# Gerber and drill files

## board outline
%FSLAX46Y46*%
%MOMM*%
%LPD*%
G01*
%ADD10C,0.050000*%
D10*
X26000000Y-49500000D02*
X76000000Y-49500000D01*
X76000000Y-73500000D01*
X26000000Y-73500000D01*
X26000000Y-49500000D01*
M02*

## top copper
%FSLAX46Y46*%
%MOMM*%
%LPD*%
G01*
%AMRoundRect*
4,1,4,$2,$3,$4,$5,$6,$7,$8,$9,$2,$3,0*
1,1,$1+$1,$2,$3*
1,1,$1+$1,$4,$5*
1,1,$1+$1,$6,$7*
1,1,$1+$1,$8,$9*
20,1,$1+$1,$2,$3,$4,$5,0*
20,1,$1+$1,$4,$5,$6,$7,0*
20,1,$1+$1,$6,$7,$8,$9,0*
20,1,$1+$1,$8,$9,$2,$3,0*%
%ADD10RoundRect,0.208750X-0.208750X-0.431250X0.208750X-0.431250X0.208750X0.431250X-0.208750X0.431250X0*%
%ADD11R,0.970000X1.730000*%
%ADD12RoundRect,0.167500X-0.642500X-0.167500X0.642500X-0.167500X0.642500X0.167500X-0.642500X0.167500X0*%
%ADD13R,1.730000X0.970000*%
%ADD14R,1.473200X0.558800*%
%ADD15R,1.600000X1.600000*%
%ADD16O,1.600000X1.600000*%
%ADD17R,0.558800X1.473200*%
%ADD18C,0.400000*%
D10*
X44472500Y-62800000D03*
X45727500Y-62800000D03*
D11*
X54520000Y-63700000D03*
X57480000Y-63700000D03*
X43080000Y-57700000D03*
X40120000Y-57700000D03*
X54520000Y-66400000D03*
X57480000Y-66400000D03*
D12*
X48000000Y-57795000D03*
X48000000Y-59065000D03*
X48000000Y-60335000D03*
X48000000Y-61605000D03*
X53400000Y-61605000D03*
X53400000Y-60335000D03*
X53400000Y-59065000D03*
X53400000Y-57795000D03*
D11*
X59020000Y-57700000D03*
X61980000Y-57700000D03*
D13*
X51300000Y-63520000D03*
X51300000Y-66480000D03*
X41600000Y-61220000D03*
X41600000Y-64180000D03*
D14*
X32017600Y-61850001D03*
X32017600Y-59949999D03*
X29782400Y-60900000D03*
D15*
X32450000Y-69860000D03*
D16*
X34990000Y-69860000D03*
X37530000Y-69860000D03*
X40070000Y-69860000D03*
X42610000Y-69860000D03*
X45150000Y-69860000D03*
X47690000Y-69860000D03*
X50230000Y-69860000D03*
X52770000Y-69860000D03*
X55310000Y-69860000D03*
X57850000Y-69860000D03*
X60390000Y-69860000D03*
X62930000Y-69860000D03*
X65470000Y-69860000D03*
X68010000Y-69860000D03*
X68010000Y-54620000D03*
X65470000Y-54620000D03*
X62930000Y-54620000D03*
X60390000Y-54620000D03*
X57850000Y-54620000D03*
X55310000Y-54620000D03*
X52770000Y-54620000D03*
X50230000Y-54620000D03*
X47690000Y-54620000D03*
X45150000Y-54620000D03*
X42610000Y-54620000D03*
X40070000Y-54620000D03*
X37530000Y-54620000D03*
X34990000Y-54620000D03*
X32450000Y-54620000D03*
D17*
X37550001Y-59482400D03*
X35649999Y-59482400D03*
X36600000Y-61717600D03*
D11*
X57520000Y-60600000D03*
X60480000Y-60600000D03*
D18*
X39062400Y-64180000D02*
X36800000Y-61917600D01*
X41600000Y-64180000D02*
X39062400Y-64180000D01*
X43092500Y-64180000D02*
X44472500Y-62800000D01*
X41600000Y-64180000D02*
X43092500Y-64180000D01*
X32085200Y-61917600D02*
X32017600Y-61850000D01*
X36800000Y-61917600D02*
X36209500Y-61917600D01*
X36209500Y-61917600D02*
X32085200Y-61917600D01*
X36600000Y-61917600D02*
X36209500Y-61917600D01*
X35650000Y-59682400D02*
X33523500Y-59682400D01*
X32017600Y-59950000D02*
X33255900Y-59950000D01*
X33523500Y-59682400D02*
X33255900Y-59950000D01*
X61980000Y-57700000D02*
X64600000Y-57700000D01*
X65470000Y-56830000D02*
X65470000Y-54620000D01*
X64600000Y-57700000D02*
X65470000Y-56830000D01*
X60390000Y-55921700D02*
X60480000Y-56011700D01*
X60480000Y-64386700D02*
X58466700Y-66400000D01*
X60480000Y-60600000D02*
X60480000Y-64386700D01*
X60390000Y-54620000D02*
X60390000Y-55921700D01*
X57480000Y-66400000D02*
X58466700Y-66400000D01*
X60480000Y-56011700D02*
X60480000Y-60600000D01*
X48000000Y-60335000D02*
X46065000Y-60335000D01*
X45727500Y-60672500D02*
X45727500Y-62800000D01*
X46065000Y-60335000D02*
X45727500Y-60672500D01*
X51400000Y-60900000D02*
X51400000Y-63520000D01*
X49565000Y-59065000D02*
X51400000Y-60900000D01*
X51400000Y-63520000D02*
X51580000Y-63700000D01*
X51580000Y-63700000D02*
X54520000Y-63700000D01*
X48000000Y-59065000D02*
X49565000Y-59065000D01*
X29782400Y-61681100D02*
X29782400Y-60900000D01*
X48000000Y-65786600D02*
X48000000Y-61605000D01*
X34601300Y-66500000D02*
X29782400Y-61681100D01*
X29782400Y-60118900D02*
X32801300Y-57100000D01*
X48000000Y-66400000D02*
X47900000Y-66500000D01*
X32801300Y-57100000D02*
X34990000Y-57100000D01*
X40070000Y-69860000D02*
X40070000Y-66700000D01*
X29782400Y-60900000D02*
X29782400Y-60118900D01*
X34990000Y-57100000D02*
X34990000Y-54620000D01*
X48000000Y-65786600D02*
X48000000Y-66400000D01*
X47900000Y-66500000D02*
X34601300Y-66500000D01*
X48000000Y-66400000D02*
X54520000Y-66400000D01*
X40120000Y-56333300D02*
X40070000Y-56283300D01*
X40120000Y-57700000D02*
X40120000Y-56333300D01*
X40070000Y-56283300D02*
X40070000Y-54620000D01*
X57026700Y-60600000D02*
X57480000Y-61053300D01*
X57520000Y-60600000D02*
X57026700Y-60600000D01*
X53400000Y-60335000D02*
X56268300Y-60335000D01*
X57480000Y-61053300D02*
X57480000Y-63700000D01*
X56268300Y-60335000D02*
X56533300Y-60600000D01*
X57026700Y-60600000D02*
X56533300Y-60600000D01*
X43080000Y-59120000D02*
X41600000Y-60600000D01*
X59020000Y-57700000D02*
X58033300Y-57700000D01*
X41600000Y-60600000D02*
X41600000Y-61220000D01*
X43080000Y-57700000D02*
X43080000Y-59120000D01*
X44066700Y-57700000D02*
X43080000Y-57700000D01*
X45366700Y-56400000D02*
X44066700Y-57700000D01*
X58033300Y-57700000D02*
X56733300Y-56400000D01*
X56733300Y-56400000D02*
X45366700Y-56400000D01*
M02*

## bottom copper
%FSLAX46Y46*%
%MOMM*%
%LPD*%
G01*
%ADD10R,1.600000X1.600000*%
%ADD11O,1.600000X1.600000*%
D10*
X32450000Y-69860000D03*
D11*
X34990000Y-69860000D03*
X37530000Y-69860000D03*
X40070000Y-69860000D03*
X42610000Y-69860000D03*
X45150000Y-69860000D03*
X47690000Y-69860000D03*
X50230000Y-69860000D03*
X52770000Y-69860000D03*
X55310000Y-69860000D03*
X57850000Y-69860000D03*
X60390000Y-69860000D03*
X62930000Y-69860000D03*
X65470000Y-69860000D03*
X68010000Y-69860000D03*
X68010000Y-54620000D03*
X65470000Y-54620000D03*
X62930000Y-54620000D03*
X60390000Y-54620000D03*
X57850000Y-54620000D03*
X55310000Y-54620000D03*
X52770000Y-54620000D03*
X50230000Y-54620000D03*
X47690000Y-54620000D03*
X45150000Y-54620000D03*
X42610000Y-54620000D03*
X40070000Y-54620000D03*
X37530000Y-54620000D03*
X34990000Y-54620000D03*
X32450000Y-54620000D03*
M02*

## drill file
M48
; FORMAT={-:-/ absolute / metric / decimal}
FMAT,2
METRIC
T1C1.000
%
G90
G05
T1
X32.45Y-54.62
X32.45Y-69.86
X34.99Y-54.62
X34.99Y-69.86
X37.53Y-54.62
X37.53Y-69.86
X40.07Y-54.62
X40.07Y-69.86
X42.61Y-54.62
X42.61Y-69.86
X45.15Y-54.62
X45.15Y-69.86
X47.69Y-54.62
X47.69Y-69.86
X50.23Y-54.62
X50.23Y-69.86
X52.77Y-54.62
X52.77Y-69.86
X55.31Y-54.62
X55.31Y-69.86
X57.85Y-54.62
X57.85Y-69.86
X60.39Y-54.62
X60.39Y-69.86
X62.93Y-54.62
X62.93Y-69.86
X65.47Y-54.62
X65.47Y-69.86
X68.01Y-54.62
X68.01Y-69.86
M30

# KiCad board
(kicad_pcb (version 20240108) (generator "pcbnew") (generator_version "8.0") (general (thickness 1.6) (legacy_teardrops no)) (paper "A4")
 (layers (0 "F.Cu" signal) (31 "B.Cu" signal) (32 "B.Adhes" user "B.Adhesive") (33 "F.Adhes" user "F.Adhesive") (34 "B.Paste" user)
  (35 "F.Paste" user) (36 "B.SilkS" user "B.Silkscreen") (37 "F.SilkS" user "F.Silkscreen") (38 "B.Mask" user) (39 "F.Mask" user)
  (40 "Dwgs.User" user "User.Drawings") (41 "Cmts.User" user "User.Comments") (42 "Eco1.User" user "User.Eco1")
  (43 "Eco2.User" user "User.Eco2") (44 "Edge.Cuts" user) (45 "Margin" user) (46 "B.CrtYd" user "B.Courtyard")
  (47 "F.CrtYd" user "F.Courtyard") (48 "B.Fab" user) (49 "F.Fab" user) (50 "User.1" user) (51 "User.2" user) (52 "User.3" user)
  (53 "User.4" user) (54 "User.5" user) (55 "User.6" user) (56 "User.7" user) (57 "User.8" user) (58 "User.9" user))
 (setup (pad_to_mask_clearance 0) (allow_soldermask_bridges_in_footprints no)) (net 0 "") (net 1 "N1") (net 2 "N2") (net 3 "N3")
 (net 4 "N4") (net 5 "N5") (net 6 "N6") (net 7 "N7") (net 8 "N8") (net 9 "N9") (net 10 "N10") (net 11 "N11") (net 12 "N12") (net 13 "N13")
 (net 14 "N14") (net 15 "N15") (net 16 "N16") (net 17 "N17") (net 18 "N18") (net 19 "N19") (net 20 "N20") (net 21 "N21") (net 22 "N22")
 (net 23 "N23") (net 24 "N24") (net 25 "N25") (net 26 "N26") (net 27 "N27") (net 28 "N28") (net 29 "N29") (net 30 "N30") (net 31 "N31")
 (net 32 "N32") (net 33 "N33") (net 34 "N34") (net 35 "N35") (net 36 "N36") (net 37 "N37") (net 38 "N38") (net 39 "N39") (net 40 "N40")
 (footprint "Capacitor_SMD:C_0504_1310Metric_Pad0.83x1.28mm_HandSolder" (layer "F.Cu") (at 45.1 62.8)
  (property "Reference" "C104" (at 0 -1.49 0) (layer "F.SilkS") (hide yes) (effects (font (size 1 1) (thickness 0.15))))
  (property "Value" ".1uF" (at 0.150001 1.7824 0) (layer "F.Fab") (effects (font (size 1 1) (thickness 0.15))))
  (pad "1" smd roundrect (at -0.6275 0) (size 0.835 1.28) (layers "F.Cu" "F.Paste" "F.Mask") (roundrect_rratio 0.25) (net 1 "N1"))
  (pad "2" smd roundrect (at 0.6275 0) (size 0.835 1.28) (layers "F.Cu" "F.Paste" "F.Mask") (roundrect_rratio 0.25) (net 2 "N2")))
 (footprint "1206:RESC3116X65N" (layer "F.Cu") (at 56 63.7)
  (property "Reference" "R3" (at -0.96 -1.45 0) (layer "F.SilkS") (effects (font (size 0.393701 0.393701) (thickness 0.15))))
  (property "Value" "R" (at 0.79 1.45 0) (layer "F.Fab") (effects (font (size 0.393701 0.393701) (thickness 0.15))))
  (pad "1" smd rect (at -1.48 0) (size 0.97 1.73) (layers "F.Cu" "F.Paste" "F.Mask") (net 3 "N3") (solder_mask_margin 0.102))
  (pad "2" smd rect (at 1.48 0) (size 0.97 1.73) (layers "F.Cu" "F.Paste" "F.Mask") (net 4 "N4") (solder_mask_margin 0.102)))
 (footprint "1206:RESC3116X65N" (layer "F.Cu") (at 41.6 57.7 180)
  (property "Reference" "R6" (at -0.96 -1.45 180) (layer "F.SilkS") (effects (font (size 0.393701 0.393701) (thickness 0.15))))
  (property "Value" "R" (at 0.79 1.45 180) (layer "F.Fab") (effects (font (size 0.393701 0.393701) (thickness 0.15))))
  (pad "1" smd rect (at -1.48 0 180) (size 0.97 1.73) (layers "F.Cu" "F.Paste" "F.Mask") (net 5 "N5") (solder_mask_margin 0.102))
  (pad "2" smd rect (at 1.48 0 180) (size 0.97 1.73) (layers "F.Cu" "F.Paste" "F.Mask") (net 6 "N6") (solder_mask_margin 0.102)))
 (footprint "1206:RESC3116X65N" (layer "F.Cu") (at 56 66.4)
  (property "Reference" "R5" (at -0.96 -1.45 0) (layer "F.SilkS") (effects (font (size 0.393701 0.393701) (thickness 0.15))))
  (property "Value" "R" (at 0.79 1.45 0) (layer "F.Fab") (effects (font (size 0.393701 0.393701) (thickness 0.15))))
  (pad "1" smd rect (at -1.48 0) (size 0.97 1.73) (layers "F.Cu" "F.Paste" "F.Mask") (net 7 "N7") (solder_mask_margin 0.102))
  (pad "2" smd rect (at 1.48 0) (size 0.97 1.73) (layers "F.Cu" "F.Paste" "F.Mask") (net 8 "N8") (solder_mask_margin 0.102)))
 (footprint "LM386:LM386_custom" (layer "F.Cu") (at 48 57.795)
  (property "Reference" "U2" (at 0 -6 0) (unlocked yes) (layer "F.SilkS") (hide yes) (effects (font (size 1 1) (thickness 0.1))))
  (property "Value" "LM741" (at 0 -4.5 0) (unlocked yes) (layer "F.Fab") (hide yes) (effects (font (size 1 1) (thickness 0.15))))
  (pad "1" smd roundrect (at 0 0) (size 1.62 0.67) (layers "F.Cu" "F.Paste" "F.Mask") (roundrect_rratio 0.25) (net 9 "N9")
   (thermal_bridge_angle 45))
  (pad "2" smd roundrect (at 0 1.27) (size 1.62 0.67) (layers "F.Cu" "F.Paste" "F.Mask") (roundrect_rratio 0.25) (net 3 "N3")
   (thermal_bridge_angle 45))
  (pad "3" smd roundrect (at 0 2.54) (size 1.62 0.67) (layers "F.Cu" "F.Paste" "F.Mask" "Eco2.User") (roundrect_rratio 0.25) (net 2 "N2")
   (thermal_bridge_angle 45))
  (pad "4" smd roundrect (at 0 3.81) (size 1.62 0.67) (layers "F.Cu" "F.Paste" "F.Mask") (roundrect_rratio 0.25) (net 7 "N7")
   (thermal_bridge_angle 45))
  (pad "5" smd roundrect (at 5.4 3.81) (size 1.62 0.67) (layers "F.Cu" "F.Paste" "F.Mask") (roundrect_rratio 0.25) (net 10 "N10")
   (thermal_bridge_angle 45))
  (pad "6" smd roundrect (at 5.4 2.54) (size 1.62 0.67) (layers "F.Cu" "F.Paste" "F.Mask") (roundrect_rratio 0.25) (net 4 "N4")
   (thermal_bridge_angle 45))
  (pad "7" smd roundrect (at 5.4 1.27) (size 1.62 0.67) (layers "F.Cu" "F.Paste" "F.Mask") (roundrect_rratio 0.25) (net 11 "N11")
   (thermal_bridge_angle 45))
  (pad "8" smd roundrect (at 5.4 0) (size 1.62 0.67) (layers "F.Cu" "F.Paste" "F.Mask") (roundrect_rratio 0.25) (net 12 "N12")
   (thermal_bridge_angle 45)))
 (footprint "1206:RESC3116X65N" (layer "F.Cu") (at 60.5 57.7)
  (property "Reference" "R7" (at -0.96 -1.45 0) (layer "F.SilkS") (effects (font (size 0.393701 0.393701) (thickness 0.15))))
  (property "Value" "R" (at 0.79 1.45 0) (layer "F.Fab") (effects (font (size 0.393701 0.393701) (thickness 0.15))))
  (pad "1" smd rect (at -1.48 0) (size 0.97 1.73) (layers "F.Cu" "F.Paste" "F.Mask") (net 5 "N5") (solder_mask_margin 0.102))
  (pad "2" smd rect (at 1.48 0) (size 0.97 1.73) (layers "F.Cu" "F.Paste" "F.Mask") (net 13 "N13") (solder_mask_margin 0.102)))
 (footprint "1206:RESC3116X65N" (layer "F.Cu") (at 51.3 65 -90)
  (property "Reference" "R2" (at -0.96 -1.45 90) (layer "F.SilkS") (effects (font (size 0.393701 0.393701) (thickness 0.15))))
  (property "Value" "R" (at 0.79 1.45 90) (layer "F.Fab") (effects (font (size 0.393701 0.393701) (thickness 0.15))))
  (pad "1" smd rect (at -1.48 0 270) (size 0.97 1.73) (layers "F.Cu" "F.Paste" "F.Mask") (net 3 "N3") (solder_mask_margin 0.102))
  (pad "2" smd rect (at 1.48 0 270) (size 0.97 1.73) (layers "F.Cu" "F.Paste" "F.Mask") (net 7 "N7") (solder_mask_margin 0.102)))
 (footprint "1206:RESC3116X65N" (layer "F.Cu") (at 41.6 62.7 -90)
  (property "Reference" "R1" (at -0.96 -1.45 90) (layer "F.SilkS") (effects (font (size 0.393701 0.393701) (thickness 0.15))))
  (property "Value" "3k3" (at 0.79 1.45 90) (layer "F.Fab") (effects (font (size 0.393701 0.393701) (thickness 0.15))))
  (pad "1" smd rect (at -1.48 0 270) (size 0.97 1.73) (layers "F.Cu" "F.Paste" "F.Mask") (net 5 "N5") (solder_mask_margin 0.102))
  (pad "2" smd rect (at 1.48 0 270) (size 0.97 1.73) (layers "F.Cu" "F.Paste" "F.Mask") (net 1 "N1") (solder_mask_margin 0.102)))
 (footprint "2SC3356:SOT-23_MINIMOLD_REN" (layer "F.Cu") (at 30.9 60.9 90)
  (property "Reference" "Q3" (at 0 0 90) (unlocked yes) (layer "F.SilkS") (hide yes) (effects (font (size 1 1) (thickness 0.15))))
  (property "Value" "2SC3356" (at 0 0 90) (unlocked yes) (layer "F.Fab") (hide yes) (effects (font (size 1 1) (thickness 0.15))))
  (pad "1" smd rect (at -0.950001 1.1176 90) (size 0.5588 1.4732) (layers "F.Cu" "F.Paste" "F.Mask") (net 1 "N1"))
  (pad "2" smd rect (at 0.950001 1.1176 90) (size 0.5588 1.4732) (layers "F.Cu" "F.Paste" "F.Mask") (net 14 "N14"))
  (pad "3" smd rect (at 0 -1.1176 90) (size 0.5588 1.4732) (layers "F.Cu" "F.Paste" "F.Mask") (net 7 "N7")))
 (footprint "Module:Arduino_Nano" (layer "F.Cu") (at 32.45 69.86 90)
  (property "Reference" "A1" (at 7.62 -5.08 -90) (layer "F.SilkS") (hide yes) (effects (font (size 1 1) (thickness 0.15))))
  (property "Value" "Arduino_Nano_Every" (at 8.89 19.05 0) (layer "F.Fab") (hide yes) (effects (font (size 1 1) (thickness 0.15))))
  (pad "1" thru_hole rect (at 0 0 90) (size 1.6 1.6) (drill 1) (layers "*.Cu" "*.Mask") (remove_unused_layers no) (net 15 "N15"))
  (pad "2" thru_hole oval (at 0 2.54 90) (size 1.6 1.6) (drill 1) (layers "*.Cu" "*.Mask") (remove_unused_layers no) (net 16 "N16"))
  (pad "3" thru_hole oval (at 0 5.08 90) (size 1.6 1.6) (drill 1) (layers "*.Cu" "*.Mask") (remove_unused_layers no) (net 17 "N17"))
  (pad "4" thru_hole oval (at 0 7.62 90) (size 1.6 1.6) (drill 1) (layers "*.Cu" "*.Mask") (remove_unused_layers no) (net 7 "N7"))
  (pad "5" thru_hole oval (at 0 10.16 90) (size 1.6 1.6) (drill 1) (layers "*.Cu" "*.Mask") (remove_unused_layers no) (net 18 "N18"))
  (pad "6" thru_hole oval (at 0 12.7 90) (size 1.6 1.6) (drill 1) (layers "*.Cu" "*.Mask") (remove_unused_layers no) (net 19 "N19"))
  (pad "7" thru_hole oval (at 0 15.24 90) (size 1.6 1.6) (drill 1) (layers "*.Cu" "*.Mask") (remove_unused_layers no) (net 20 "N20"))
  (pad "8" thru_hole oval (at 0 17.78 90) (size 1.6 1.6) (drill 1) (layers "*.Cu" "*.Mask") (remove_unused_layers no) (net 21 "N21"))
  (pad "9" thru_hole oval (at 0 20.32 90) (size 1.6 1.6) (drill 1) (layers "*.Cu" "*.Mask") (remove_unused_layers no) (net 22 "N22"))
  (pad "10" thru_hole oval (at 0 22.86 90) (size 1.6 1.6) (drill 1) (layers "*.Cu" "*.Mask") (remove_unused_layers no) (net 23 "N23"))
  (pad "11" thru_hole oval (at 0 25.4 90) (size 1.6 1.6) (drill 1) (layers "*.Cu" "*.Mask") (remove_unused_layers no) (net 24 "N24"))
  (pad "12" thru_hole oval (at 0 27.94 90) (size 1.6 1.6) (drill 1) (layers "*.Cu" "*.Mask") (remove_unused_layers no) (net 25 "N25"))
  (pad "13" thru_hole oval (at 0 30.48 90) (size 1.6 1.6) (drill 1) (layers "*.Cu" "*.Mask") (remove_unused_layers no) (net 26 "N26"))
  (pad "14" thru_hole oval (at 0 33.02 90) (size 1.6 1.6) (drill 1) (layers "*.Cu" "*.Mask") (remove_unused_layers no) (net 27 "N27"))
  (pad "15" thru_hole oval (at 0 35.56 90) (size 1.6 1.6) (drill 1) (layers "*.Cu" "*.Mask") (remove_unused_layers no) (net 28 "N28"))
  (pad "16" thru_hole oval (at 15.24 35.56 90) (size 1.6 1.6) (drill 1) (layers "*.Cu" "*.Mask") (remove_unused_layers no) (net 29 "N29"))
  (pad "17" thru_hole oval (at 15.24 33.02 90) (size 1.6 1.6) (drill 1) (layers "*.Cu" "*.Mask") (remove_unused_layers no) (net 13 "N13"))
  (pad "18" thru_hole oval (at 15.24 30.48 90) (size 1.6 1.6) (drill 1) (layers "*.Cu" "*.Mask") (remove_unused_layers no) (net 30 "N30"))
  (pad "19" thru_hole oval (at 15.24 27.94 90) (size 1.6 1.6) (drill 1) (layers "*.Cu" "*.Mask") (remove_unused_layers no) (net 8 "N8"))
  (pad "20" thru_hole oval (at 15.24 25.4 90) (size 1.6 1.6) (drill 1) (layers "*.Cu" "*.Mask") (remove_unused_layers no) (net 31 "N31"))
  (pad "21" thru_hole oval (at 15.24 22.86 90) (size 1.6 1.6) (drill 1) (layers "*.Cu" "*.Mask") (remove_unused_layers no) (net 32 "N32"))
  (pad "22" thru_hole oval (at 15.24 20.32 90) (size 1.6 1.6) (drill 1) (layers "*.Cu" "*.Mask") (remove_unused_layers no) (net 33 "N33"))
  (pad "23" thru_hole oval (at 15.24 17.78 90) (size 1.6 1.6) (drill 1) (layers "*.Cu" "*.Mask") (remove_unused_layers no) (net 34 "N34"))
  (pad "24" thru_hole oval (at 15.24 15.24 90) (size 1.6 1.6) (drill 1) (layers "*.Cu" "*.Mask") (remove_unused_layers no) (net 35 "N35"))
  (pad "25" thru_hole oval (at 15.24 12.7 90) (size 1.6 1.6) (drill 1) (layers "*.Cu" "*.Mask") (remove_unused_layers no) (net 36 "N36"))
  (pad "26" thru_hole oval (at 15.24 10.16 90) (size 1.6 1.6) (drill 1) (layers "*.Cu" "*.Mask") (remove_unused_layers no) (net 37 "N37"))
  (pad "27" thru_hole oval (at 15.24 7.62 90) (size 1.6 1.6) (drill 1) (layers "*.Cu" "*.Mask") (remove_unused_layers no) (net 6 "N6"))
  (pad "28" thru_hole oval (at 15.24 5.08 90) (size 1.6 1.6) (drill 1) (layers "*.Cu" "*.Mask") (remove_unused_layers no) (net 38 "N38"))
  (pad "29" thru_hole oval (at 15.24 2.54 90) (size 1.6 1.6) (drill 1) (layers "*.Cu" "*.Mask") (remove_unused_layers no) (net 7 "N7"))
  (pad "30" thru_hole oval (at 15.24 0 90) (size 1.6 1.6) (drill 1) (layers "*.Cu" "*.Mask") (remove_unused_layers no) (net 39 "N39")))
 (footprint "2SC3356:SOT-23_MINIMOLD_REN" (layer "F.Cu") (at 36.6 60.6 180)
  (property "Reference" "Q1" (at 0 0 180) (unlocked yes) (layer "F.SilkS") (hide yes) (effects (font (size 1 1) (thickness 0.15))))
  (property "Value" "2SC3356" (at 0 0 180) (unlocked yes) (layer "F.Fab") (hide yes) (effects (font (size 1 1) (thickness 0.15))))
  (pad "1" smd rect (at -0.950001 1.1176 180) (size 0.5588 1.4732) (layers "F.Cu" "F.Paste" "F.Mask") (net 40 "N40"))
  (pad "2" smd rect (at 0.950001 1.1176 180) (size 0.5588 1.4732) (layers "F.Cu" "F.Paste" "F.Mask") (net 14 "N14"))
  (pad "3" smd rect (at 0 -1.1176 180) (size 0.5588 1.4732) (layers "F.Cu" "F.Paste" "F.Mask") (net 1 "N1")))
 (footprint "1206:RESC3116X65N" (layer "F.Cu") (at 59 60.6)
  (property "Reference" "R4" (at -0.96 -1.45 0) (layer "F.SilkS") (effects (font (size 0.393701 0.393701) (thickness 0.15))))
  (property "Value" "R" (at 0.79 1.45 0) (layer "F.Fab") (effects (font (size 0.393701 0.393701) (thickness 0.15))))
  (pad "1" smd rect (at -1.48 0) (size 0.97 1.73) (layers "F.Cu" "F.Paste" "F.Mask") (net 4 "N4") (solder_mask_margin 0.102))
  (pad "2" smd rect (at 1.48 0) (size 0.97 1.73) (layers "F.Cu" "F.Paste" "F.Mask") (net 8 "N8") (solder_mask_margin 0.102)))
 (gr_rect (start 26 49.5) (end 76 73.5) (stroke (width 0.05) (type default)) (fill none) (layer "Edge.Cuts"))
 (segment (start 39.0624 64.18) (end 36.8 61.9176) (width 0.4) (layer "F.Cu") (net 1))
 (segment (start 41.6 64.18) (end 39.0624 64.18) (width 0.4) (layer "F.Cu") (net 1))
 (segment (start 43.0925 64.18) (end 44.4725 62.8) (width 0.4) (layer "F.Cu") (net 1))
 (segment (start 41.6 64.18) (end 43.0925 64.18) (width 0.4) (layer "F.Cu") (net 1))
 (segment (start 32.0852 61.9176) (end 32.0176 61.85) (width 0.4) (layer "F.Cu") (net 1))
 (segment (start 36.8 61.9176) (end 36.2095 61.9176) (width 0.4) (layer "F.Cu") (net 1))
 (segment (start 36.2095 61.9176) (end 32.0852 61.9176) (width 0.4) (layer "F.Cu") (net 1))
 (segment (start 36.6 61.9176) (end 36.2095 61.9176) (width 0.4) (layer "F.Cu") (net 1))
 (segment (start 35.65 59.6824) (end 33.5235 59.6824) (width 0.4) (layer "F.Cu") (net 14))
 (segment (start 32.0176 59.95) (end 33.2559 59.95) (width 0.4) (layer "F.Cu") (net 14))
 (segment (start 33.5235 59.6824) (end 33.2559 59.95) (width 0.4) (layer "F.Cu") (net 14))
 (segment (start 61.98 57.7) (end 64.6 57.7) (width 0.4) (layer "F.Cu") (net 13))
 (segment (start 65.47 56.83) (end 65.47 54.62) (width 0.4) (layer "F.Cu") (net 13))
 (segment (start 64.6 57.7) (end 65.47 56.83) (width 0.4) (layer "F.Cu") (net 13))
 (segment (start 60.39 55.9217) (end 60.48 56.0117) (width 0.4) (layer "F.Cu") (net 8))
 (segment (start 60.48 64.3867) (end 58.4667 66.4) (width 0.4) (layer "F.Cu") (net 8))
 (segment (start 60.48 60.6) (end 60.48 64.3867) (width 0.4) (layer "F.Cu") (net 8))
 (segment (start 60.39 54.62) (end 60.39 55.9217) (width 0.4) (layer "F.Cu") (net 8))
 (segment (start 57.48 66.4) (end 58.4667 66.4) (width 0.4) (layer "F.Cu") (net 8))
 (segment (start 60.48 56.0117) (end 60.48 60.6) (width 0.4) (layer "F.Cu") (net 8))
 (segment (start 48 60.335) (end 46.065 60.335) (width 0.4) (layer "F.Cu") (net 2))
 (segment (start 45.7275 60.6725) (end 45.7275 62.8) (width 0.4) (layer "F.Cu") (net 2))
 (segment (start 46.065 60.335) (end 45.7275 60.6725) (width 0.4) (layer "F.Cu") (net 2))
 (segment (start 51.4 60.9) (end 51.4 63.52) (width 0.4) (layer "F.Cu") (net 3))
 (segment (start 49.565 59.065) (end 51.4 60.9) (width 0.4) (layer "F.Cu") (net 3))
 (segment (start 51.4 63.52) (end 51.58 63.7) (width 0.4) (layer "F.Cu") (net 3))
 (segment (start 51.58 63.7) (end 54.52 63.7) (width 0.4) (layer "F.Cu") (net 3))
 (segment (start 48 59.065) (end 49.565 59.065) (width 0.4) (layer "F.Cu") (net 3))
 (segment (start 29.7824 61.6811) (end 29.7824 60.9) (width 0.4) (layer "F.Cu") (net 7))
 (segment (start 48 65.7866) (end 48 61.605) (width 0.4) (layer "F.Cu") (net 7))
 (segment (start 34.6013 66.5) (end 29.7824 61.6811) (width 0.4) (layer "F.Cu") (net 7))
 (segment (start 29.7824 60.1189) (end 32.8013 57.1) (width 0.4) (layer "F.Cu") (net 7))
 (segment (start 48 66.4) (end 47.9 66.5) (width 0.4) (layer "F.Cu") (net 7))
 (segment (start 32.8013 57.1) (end 34.99 57.1) (width 0.4) (layer "F.Cu") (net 7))
 (segment (start 40.07 69.86) (end 40.07 66.7) (width 0.4) (layer "F.Cu") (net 7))
 (segment (start 29.7824 60.9) (end 29.7824 60.1189) (width 0.4) (layer "F.Cu") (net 7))
 (segment (start 34.99 57.1) (end 34.99 54.62) (width 0.4) (layer "F.Cu") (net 7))
 (segment (start 48 65.7866) (end 48 66.4) (width 0.4) (layer "F.Cu") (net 7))
 (segment (start 47.9 66.5) (end 34.6013 66.5) (width 0.4) (layer "F.Cu") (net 7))
 (segment (start 48 66.4) (end 54.52 66.4) (width 0.4) (layer "F.Cu") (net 7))
 (segment (start 40.12 56.3333) (end 40.07 56.2833) (width 0.4) (layer "F.Cu") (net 6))
 (segment (start 40.12 57.7) (end 40.12 56.3333) (width 0.4) (layer "F.Cu") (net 6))
 (segment (start 40.07 56.2833) (end 40.07 54.62) (width 0.4) (layer "F.Cu") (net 6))
 (segment (start 57.0267 60.6) (end 57.48 61.0533) (width 0.4) (layer "F.Cu") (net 4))
 (segment (start 57.52 60.6) (end 57.0267 60.6) (width 0.4) (layer "F.Cu") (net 4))
 (segment (start 53.4 60.335) (end 56.2683 60.335) (width 0.4) (layer "F.Cu") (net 4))
 (segment (start 57.48 61.0533) (end 57.48 63.7) (width 0.4) (layer "F.Cu") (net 4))
 (segment (start 56.2683 60.335) (end 56.5333 60.6) (width 0.4) (layer "F.Cu") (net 4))
 (segment (start 57.0267 60.6) (end 56.5333 60.6) (width 0.4) (layer "F.Cu") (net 4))
 (segment (start 43.08 59.12) (end 41.6 60.6) (width 0.4) (layer "F.Cu") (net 5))
 (segment (start 59.02 57.7) (end 58.0333 57.7) (width 0.4) (layer "F.Cu") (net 5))
 (segment (start 41.6 60.6) (end 41.6 61.22) (width 0.4) (layer "F.Cu") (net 5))
 (segment (start 43.08 57.7) (end 43.08 59.12) (width 0.4) (layer "F.Cu") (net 5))
 (segment (start 44.0667 57.7) (end 43.08 57.7) (width 0.4) (layer "F.Cu") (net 5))
 (segment (start 45.3667 56.4) (end 44.0667 57.7) (width 0.4) (layer "F.Cu") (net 5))
 (segment (start 58.0333 57.7) (end 56.7333 56.4) (width 0.4) (layer "F.Cu") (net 5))
 (segment (start 56.7333 56.4) (end 45.3667 56.4) (width 0.4) (layer "F.Cu") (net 5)))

